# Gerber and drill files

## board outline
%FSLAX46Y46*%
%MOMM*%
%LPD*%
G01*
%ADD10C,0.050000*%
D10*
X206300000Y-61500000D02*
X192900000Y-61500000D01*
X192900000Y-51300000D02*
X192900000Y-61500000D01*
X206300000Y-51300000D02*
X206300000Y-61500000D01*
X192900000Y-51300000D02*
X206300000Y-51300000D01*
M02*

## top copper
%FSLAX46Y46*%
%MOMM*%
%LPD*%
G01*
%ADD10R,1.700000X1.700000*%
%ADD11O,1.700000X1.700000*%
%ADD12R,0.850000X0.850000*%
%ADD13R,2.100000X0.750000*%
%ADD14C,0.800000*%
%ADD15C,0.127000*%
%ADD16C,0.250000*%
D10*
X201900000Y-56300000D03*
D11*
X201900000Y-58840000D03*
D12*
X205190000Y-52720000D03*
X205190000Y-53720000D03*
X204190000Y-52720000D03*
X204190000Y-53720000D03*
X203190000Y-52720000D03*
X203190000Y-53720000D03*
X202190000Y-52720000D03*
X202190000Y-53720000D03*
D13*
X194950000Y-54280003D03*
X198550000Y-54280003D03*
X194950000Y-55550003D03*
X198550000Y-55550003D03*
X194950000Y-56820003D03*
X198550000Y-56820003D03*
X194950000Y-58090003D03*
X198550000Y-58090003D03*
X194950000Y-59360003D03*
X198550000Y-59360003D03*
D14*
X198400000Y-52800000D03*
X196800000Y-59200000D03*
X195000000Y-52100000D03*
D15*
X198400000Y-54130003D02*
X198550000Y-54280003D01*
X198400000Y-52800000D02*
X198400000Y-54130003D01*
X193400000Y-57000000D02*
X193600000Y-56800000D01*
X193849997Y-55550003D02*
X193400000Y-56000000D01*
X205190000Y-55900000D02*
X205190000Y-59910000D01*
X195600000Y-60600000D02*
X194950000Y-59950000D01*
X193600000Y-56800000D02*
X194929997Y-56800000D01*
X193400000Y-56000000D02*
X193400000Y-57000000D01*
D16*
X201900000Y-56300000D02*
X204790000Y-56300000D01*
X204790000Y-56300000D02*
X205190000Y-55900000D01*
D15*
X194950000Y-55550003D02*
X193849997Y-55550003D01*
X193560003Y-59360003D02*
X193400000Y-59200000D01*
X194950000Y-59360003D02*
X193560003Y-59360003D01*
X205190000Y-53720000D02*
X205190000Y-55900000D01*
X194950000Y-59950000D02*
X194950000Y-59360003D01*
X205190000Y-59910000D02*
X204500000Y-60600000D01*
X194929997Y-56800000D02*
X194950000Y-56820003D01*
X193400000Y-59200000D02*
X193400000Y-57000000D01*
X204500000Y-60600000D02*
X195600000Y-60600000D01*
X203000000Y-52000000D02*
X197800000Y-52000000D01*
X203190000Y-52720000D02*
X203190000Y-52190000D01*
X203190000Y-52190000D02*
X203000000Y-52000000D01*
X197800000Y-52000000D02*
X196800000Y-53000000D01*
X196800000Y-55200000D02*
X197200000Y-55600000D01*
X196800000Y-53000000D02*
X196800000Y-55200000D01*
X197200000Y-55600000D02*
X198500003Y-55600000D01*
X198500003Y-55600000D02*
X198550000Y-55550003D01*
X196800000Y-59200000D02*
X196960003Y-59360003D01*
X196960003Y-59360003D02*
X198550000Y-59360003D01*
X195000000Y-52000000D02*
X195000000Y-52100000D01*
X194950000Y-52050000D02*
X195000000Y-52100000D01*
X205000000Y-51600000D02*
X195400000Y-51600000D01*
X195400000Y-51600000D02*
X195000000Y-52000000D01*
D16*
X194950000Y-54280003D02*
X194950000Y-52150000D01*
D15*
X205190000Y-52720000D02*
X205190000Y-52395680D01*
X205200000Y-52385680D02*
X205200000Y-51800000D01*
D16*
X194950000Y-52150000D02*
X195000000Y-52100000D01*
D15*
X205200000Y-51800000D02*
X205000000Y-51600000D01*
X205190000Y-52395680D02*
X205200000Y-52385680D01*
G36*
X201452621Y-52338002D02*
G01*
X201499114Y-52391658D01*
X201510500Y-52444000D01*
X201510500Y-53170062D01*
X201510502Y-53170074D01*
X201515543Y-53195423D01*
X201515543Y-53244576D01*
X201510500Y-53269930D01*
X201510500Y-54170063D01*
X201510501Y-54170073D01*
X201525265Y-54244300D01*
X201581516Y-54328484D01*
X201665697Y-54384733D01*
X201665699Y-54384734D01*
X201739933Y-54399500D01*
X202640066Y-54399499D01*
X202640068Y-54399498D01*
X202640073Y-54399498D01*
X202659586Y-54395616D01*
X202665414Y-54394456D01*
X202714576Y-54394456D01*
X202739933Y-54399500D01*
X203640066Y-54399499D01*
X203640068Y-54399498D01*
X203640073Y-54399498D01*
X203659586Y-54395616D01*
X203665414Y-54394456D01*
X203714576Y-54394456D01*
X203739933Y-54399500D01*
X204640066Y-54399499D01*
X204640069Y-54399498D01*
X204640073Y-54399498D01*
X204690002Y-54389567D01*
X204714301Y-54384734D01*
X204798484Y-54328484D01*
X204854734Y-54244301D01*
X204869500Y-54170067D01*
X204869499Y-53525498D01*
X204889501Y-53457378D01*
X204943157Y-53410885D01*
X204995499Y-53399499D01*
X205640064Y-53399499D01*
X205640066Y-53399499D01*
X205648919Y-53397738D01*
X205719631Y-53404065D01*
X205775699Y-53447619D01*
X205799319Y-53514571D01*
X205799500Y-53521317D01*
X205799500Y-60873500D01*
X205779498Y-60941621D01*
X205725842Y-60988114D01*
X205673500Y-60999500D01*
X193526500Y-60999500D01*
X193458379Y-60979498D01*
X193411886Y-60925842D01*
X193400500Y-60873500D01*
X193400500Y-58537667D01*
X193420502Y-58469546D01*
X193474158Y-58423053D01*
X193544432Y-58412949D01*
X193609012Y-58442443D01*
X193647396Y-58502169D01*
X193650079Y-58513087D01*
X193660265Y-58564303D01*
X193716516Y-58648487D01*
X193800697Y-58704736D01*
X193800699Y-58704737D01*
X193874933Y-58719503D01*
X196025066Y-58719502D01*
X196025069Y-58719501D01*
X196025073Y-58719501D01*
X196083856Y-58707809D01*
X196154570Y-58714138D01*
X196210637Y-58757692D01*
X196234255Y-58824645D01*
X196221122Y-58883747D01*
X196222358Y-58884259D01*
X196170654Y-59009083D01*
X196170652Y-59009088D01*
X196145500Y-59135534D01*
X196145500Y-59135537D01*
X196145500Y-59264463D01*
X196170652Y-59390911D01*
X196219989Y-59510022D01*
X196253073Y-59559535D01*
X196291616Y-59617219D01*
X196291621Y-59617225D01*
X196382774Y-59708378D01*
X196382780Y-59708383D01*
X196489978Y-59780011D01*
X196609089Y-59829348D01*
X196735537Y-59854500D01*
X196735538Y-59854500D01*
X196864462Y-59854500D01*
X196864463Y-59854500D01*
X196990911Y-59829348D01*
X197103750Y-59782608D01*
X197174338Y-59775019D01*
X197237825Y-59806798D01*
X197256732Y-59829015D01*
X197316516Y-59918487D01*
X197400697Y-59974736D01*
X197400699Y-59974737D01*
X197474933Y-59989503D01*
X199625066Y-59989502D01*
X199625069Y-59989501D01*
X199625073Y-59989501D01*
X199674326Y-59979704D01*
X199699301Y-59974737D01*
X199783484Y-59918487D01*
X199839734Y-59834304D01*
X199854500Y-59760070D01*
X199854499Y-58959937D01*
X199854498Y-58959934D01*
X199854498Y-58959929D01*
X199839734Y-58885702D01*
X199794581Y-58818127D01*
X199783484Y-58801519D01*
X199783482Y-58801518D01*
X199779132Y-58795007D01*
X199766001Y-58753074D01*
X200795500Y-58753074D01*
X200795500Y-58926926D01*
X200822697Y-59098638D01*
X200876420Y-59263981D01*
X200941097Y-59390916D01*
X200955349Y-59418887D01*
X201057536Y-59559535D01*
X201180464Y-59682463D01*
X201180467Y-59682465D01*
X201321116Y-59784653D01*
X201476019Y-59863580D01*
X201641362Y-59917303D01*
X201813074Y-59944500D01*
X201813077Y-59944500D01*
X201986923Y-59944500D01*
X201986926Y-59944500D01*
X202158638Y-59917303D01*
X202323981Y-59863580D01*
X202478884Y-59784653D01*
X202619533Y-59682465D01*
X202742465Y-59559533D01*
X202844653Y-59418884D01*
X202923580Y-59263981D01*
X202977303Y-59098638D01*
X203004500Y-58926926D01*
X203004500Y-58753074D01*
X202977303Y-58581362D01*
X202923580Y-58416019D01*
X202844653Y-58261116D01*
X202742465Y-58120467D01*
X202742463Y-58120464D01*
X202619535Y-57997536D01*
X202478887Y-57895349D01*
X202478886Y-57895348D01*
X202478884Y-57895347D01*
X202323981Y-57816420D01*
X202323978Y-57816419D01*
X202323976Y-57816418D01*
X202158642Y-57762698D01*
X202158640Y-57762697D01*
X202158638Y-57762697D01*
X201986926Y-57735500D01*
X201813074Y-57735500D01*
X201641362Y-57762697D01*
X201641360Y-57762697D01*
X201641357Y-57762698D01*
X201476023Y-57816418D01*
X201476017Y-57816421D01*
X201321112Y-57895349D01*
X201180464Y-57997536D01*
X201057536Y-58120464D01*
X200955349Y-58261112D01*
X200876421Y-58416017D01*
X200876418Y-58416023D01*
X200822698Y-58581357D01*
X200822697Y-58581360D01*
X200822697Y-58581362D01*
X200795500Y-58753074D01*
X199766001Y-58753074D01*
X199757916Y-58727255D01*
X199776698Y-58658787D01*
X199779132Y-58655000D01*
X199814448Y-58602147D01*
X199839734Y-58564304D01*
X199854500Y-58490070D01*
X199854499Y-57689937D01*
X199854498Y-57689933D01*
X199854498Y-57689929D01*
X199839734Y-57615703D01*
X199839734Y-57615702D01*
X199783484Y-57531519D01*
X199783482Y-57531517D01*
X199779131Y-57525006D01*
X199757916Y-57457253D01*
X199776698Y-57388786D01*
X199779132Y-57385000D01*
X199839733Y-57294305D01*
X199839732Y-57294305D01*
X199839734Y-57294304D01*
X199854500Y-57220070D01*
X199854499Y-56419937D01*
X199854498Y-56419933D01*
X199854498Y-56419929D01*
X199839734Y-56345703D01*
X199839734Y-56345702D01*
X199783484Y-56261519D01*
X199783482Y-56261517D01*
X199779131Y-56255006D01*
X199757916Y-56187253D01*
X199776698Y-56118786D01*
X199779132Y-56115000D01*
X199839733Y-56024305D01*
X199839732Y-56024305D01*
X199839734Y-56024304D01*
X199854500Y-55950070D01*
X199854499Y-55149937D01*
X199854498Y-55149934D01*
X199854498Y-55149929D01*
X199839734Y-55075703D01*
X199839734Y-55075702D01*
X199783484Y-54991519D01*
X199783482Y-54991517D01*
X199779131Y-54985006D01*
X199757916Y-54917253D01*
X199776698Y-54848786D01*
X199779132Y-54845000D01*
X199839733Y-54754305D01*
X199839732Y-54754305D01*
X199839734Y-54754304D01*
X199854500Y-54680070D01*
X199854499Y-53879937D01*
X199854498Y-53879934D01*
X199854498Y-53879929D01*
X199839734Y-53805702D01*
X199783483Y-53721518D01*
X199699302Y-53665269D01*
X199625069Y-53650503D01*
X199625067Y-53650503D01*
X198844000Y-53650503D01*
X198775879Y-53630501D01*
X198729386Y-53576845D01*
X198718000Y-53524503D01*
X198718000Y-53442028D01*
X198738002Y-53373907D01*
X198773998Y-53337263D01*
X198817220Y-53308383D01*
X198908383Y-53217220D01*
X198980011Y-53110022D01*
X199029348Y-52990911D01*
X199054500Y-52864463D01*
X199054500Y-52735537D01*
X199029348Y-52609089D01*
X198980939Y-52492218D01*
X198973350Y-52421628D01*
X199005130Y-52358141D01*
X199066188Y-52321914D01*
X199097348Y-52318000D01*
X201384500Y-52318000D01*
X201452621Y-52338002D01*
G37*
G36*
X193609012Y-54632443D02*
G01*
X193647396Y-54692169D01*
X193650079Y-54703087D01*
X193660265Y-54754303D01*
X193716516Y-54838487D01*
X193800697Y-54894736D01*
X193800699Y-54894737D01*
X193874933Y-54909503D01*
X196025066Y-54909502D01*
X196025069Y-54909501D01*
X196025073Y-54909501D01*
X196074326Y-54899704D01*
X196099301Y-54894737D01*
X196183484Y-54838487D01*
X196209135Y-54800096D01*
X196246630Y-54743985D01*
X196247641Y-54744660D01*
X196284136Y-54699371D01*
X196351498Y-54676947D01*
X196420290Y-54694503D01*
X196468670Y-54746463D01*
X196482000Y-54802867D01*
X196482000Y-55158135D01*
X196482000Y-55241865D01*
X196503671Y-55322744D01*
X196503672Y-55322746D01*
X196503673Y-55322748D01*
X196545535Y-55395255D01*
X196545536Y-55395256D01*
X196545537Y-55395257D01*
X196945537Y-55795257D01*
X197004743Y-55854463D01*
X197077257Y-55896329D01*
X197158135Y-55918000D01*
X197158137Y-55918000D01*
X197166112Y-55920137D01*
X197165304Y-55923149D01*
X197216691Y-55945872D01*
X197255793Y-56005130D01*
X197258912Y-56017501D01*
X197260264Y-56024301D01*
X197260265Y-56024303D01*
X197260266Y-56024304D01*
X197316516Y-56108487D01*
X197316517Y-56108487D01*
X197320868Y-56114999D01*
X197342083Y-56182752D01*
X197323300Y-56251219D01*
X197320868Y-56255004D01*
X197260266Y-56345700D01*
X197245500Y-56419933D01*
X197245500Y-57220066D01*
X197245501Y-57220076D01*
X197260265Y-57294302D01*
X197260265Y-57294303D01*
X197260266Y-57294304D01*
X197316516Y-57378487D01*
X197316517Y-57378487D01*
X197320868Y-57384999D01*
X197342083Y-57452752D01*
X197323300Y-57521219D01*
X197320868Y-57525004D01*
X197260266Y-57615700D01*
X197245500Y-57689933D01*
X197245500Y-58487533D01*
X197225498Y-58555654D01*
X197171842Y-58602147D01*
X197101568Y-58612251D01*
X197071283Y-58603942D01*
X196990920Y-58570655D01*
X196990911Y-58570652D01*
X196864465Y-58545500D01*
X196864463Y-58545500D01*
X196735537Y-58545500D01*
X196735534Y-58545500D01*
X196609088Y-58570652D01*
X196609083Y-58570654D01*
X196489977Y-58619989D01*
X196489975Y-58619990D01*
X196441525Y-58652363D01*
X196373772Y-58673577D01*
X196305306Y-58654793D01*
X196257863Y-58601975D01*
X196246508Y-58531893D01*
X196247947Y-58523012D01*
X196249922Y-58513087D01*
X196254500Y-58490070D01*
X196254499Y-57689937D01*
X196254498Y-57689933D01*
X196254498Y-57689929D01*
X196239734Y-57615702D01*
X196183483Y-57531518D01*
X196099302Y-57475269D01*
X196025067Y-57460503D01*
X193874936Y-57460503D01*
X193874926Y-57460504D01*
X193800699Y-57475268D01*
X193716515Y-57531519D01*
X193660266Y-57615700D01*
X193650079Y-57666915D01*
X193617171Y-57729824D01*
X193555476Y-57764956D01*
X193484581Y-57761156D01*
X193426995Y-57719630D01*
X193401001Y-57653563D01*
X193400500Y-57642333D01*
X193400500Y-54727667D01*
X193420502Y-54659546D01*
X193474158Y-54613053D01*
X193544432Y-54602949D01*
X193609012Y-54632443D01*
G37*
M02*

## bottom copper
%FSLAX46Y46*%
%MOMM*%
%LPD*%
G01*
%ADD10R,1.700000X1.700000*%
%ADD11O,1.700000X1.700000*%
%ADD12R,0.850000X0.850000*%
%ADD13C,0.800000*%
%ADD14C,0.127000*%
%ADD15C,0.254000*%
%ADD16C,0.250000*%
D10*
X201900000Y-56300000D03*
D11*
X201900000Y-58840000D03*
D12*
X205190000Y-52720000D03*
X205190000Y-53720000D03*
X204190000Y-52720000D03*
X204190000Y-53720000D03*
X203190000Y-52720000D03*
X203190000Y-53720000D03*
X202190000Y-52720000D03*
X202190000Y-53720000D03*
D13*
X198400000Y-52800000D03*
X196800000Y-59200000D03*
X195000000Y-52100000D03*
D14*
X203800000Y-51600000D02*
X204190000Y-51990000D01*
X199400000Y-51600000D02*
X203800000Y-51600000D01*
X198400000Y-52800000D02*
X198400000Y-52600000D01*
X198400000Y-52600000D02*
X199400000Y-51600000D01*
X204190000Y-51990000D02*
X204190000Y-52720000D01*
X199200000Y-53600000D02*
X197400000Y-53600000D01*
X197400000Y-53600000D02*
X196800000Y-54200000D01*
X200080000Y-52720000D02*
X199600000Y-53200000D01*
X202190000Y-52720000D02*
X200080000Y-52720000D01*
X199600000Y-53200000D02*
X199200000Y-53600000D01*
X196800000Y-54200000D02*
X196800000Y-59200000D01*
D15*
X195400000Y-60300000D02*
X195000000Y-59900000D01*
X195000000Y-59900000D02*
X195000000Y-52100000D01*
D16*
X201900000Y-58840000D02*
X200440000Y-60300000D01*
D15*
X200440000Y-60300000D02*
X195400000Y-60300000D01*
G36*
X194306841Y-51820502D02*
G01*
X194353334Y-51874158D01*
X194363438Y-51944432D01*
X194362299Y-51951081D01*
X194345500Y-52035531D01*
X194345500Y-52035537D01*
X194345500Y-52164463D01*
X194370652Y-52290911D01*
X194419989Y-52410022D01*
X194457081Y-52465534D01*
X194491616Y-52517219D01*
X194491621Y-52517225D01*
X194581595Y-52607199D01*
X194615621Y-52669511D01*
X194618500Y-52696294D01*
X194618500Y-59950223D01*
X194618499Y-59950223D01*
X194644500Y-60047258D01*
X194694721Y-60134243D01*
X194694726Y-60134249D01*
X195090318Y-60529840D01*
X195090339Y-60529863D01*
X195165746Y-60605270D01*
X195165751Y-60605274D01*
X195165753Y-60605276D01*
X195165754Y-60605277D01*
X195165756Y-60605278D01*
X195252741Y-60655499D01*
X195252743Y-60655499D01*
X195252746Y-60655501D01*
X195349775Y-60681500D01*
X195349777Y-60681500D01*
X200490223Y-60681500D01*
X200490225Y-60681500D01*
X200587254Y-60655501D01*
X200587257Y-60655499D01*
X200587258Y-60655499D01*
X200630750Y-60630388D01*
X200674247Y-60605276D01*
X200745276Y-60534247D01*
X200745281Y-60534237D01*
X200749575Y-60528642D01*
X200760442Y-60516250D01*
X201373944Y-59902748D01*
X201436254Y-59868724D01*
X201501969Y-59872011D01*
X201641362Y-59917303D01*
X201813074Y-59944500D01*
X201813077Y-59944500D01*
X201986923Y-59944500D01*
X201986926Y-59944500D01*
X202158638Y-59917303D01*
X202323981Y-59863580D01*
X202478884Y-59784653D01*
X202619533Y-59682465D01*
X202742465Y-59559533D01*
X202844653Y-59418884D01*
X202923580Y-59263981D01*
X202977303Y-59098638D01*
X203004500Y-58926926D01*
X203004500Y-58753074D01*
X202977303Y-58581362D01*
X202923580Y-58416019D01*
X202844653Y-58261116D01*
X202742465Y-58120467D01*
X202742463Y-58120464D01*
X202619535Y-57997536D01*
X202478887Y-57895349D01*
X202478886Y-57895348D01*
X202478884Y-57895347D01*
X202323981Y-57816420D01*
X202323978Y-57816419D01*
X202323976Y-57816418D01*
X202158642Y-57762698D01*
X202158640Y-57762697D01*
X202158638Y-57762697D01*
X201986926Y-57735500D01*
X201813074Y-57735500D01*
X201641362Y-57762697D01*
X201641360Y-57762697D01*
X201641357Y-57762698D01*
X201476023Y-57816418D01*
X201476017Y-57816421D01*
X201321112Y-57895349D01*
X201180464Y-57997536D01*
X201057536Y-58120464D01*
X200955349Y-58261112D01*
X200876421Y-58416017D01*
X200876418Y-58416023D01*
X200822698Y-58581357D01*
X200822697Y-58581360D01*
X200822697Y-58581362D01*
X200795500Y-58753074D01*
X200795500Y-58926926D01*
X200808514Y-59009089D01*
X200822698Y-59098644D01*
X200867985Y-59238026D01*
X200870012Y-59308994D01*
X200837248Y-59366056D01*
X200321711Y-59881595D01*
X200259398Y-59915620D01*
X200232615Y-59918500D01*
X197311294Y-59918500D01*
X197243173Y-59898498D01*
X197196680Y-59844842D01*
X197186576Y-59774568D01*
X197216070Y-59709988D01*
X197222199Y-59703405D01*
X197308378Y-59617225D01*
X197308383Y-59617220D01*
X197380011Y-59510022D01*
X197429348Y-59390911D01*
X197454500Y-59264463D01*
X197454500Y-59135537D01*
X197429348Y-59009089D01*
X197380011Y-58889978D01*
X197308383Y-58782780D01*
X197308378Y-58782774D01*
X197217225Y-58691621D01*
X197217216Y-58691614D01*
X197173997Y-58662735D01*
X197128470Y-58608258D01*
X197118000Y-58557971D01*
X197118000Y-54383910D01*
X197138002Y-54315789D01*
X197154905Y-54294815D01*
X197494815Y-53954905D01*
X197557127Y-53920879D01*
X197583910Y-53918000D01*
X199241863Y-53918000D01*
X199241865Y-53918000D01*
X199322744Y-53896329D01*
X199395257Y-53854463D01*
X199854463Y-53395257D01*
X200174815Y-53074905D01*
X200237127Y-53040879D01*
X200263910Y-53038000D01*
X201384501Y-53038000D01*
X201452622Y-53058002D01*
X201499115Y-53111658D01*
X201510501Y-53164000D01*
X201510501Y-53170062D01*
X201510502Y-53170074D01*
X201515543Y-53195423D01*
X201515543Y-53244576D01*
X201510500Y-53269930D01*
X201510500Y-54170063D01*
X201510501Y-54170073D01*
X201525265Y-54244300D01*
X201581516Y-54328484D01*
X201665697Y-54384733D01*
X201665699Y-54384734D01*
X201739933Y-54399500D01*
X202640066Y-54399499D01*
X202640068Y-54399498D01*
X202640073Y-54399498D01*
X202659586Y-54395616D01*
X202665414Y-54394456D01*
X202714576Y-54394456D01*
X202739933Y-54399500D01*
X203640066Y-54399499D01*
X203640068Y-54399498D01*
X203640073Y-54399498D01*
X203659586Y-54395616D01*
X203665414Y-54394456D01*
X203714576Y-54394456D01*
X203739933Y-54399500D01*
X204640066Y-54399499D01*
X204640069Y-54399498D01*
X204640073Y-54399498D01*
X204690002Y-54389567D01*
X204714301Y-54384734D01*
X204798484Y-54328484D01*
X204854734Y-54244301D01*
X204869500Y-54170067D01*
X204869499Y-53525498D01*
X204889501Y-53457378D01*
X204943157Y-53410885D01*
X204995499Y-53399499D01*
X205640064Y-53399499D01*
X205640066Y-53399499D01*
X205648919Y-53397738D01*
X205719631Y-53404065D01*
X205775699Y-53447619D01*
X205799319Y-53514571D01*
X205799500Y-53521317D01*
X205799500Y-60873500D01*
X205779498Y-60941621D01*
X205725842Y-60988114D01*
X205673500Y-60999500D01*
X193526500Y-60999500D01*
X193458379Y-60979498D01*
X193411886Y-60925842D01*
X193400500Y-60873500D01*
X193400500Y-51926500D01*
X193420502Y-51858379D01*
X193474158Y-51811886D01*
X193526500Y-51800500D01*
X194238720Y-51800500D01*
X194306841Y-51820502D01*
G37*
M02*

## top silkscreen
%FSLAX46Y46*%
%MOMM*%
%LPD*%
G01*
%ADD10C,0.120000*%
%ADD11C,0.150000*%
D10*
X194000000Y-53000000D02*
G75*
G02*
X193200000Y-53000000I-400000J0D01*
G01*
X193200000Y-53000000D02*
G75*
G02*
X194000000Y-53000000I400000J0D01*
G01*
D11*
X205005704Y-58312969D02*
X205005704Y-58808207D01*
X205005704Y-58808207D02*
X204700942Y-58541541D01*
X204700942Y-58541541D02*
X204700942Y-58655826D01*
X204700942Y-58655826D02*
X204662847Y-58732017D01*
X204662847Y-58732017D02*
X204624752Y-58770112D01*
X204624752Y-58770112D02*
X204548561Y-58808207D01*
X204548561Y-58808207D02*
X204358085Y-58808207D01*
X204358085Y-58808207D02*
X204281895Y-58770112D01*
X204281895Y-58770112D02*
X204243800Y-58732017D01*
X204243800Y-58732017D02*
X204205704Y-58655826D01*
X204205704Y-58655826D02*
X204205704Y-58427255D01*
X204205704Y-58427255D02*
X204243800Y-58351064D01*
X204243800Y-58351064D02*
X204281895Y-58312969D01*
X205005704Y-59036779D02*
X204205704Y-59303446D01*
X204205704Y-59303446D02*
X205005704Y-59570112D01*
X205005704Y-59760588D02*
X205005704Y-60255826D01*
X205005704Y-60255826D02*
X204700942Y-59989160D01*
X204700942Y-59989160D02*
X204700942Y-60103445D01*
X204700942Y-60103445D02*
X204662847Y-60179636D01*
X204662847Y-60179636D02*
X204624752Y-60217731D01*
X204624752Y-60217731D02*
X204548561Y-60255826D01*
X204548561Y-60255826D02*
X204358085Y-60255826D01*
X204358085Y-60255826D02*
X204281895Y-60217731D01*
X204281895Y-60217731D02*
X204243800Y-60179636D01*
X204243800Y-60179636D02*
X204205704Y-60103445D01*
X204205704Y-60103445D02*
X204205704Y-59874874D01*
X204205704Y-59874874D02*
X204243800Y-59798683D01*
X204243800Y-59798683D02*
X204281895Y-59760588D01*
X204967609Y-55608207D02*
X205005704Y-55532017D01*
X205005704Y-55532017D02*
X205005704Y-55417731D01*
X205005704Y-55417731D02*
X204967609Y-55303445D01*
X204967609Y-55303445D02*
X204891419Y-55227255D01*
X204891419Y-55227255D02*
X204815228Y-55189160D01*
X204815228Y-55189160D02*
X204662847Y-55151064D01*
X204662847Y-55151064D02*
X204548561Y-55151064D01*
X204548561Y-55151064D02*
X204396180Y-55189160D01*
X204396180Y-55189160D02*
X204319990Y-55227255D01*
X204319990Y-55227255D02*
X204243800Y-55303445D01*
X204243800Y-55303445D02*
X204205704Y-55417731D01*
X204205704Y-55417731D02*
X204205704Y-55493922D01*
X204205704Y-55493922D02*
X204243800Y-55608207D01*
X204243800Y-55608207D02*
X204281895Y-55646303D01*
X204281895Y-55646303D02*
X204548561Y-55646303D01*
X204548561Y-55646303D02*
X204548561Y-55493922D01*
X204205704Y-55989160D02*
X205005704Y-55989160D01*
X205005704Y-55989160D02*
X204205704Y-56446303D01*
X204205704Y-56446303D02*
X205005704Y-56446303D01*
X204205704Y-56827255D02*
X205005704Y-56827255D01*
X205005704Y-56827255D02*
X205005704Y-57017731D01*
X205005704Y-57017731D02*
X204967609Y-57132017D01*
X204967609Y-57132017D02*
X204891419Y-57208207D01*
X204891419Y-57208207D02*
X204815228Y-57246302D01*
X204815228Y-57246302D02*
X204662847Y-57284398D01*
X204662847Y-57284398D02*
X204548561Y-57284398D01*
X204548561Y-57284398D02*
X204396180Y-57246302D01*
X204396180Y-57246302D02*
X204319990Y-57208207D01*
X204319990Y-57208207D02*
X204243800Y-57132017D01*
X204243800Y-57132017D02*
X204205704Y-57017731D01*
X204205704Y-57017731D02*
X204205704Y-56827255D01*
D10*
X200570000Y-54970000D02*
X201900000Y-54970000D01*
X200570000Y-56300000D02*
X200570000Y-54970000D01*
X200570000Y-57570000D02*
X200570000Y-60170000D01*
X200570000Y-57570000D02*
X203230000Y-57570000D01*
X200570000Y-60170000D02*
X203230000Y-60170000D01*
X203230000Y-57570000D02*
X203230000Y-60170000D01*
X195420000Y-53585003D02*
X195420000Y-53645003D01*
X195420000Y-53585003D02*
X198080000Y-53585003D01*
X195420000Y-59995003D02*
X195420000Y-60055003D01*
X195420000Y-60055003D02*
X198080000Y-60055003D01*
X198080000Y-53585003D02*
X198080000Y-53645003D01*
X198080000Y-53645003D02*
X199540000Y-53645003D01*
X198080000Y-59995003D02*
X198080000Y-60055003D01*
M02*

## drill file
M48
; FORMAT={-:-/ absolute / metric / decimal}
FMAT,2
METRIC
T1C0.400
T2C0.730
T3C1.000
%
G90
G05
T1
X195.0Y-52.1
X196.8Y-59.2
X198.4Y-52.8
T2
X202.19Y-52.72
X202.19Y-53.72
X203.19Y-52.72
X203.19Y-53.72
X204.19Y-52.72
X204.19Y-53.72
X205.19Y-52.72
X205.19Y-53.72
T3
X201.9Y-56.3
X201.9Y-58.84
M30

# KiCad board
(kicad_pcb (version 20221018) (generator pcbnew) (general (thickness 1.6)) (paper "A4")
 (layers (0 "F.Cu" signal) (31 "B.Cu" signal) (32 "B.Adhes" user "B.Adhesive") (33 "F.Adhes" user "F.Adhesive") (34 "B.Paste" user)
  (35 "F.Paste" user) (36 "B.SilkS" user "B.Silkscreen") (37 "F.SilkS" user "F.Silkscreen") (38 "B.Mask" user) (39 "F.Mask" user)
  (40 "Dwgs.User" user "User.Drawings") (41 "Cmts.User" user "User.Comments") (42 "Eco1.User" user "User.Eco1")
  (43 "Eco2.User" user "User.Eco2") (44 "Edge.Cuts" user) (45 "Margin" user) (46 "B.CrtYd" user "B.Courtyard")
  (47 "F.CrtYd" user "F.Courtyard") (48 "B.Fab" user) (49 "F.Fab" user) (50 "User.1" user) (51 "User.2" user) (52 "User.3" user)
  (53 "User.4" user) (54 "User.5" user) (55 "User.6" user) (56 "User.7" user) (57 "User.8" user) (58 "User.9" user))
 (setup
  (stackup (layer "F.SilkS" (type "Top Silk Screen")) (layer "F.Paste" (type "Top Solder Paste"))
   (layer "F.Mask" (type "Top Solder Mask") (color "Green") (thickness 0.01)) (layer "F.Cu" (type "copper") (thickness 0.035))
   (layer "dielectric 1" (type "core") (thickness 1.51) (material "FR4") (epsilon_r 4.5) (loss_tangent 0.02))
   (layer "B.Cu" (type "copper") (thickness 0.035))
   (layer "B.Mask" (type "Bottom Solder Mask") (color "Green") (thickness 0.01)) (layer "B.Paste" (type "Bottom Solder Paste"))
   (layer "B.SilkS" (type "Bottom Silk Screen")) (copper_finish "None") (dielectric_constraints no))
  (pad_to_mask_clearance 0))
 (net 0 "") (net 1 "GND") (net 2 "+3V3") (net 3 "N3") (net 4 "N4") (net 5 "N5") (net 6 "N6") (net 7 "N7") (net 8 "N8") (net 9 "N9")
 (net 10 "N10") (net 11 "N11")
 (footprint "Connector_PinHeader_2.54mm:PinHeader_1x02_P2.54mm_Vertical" (layer "F.Cu") (at 201.9 56.3)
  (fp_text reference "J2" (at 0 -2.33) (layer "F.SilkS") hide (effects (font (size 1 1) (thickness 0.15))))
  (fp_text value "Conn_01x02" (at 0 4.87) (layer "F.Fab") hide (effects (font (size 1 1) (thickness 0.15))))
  (fp_line (start -1.33 -1.33) (end 0 -1.33) (stroke (width 0.12) (type solid)) (layer "F.SilkS"))
  (fp_line (start -1.33 0) (end -1.33 -1.33) (stroke (width 0.12) (type solid)) (layer "F.SilkS"))
  (fp_line (start -1.33 1.27) (end -1.33 3.87) (stroke (width 0.12) (type solid)) (layer "F.SilkS"))
  (fp_line (start -1.33 1.27) (end 1.33 1.27) (stroke (width 0.12) (type solid)) (layer "F.SilkS"))
  (fp_line (start -1.33 3.87) (end 1.33 3.87) (stroke (width 0.12) (type solid)) (layer "F.SilkS"))
  (fp_line (start 1.33 1.27) (end 1.33 3.87) (stroke (width 0.12) (type solid)) (layer "F.SilkS"))
  (pad "1" thru_hole rect (at 0 0) (size 1.7 1.7) (drill 1) (layers "*.Cu" "*.Mask") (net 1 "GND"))
  (pad "2" thru_hole oval (at 0 2.54) (size 1.7 1.7) (drill 1) (layers "*.Cu" "*.Mask") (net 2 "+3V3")))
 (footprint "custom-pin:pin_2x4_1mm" (layer "F.Cu") (at 203.69 53.22)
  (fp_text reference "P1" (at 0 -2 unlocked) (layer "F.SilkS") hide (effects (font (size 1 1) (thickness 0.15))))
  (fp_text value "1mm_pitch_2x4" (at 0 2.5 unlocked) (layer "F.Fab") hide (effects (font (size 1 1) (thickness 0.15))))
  (pad "1" thru_hole rect (at 1.5 -0.5) (size 0.85 0.85) (drill 0.73) (layers "*.Cu" "*.Mask") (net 2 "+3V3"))
  (pad "2" thru_hole rect (at 1.5 0.5) (size 0.85 0.85) (drill 0.73) (layers "*.Cu" "*.Mask") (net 1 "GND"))
  (pad "3" thru_hole rect (at 0.5 -0.5) (size 0.85 0.85) (drill 0.73) (layers "*.Cu" "*.Mask") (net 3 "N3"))
  (pad "4" thru_hole rect (at 0.5 0.5) (size 0.85 0.85) (drill 0.73) (layers "*.Cu" "*.Mask") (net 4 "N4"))
  (pad "5" thru_hole rect (at -0.5 -0.5) (size 0.85 0.85) (drill 0.73) (layers "*.Cu" "*.Mask") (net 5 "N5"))
  (pad "6" thru_hole rect (at -0.5 0.5) (size 0.85 0.85) (drill 0.73) (layers "*.Cu" "*.Mask") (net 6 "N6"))
  (pad "7" thru_hole rect (at -1.5 -0.5) (size 0.85 0.85) (drill 0.73) (layers "*.Cu" "*.Mask") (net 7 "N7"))
  (pad "8" thru_hole rect (at -1.5 0.5) (size 0.85 0.85) (drill 0.73) (layers "*.Cu" "*.Mask") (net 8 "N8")))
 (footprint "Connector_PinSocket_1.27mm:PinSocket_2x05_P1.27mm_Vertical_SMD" (layer "F.Cu") (at 196.75 56.820003)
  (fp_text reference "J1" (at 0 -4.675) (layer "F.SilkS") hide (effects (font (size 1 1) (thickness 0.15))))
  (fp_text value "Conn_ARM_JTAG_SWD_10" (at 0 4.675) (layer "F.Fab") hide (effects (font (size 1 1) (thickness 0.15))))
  (fp_line (start -1.33 -3.235) (end -1.33 -3.175) (stroke (width 0.12) (type solid)) (layer "F.SilkS"))
  (fp_line (start -1.33 -3.235) (end 1.33 -3.235) (stroke (width 0.12) (type solid)) (layer "F.SilkS"))
  (fp_line (start -1.33 3.175) (end -1.33 3.235) (stroke (width 0.12) (type solid)) (layer "F.SilkS"))
  (fp_line (start -1.33 3.235) (end 1.33 3.235) (stroke (width 0.12) (type solid)) (layer "F.SilkS"))
  (fp_line (start 1.33 -3.235) (end 1.33 -3.175) (stroke (width 0.12) (type solid)) (layer "F.SilkS"))
  (fp_line (start 1.33 -3.175) (end 2.79 -3.175) (stroke (width 0.12) (type solid)) (layer "F.SilkS"))
  (fp_line (start 1.33 3.175) (end 1.33 3.235) (stroke (width 0.12) (type solid)) (layer "F.SilkS"))
  (pad "1" smd rect (at -1.8 -2.54) (size 2.1 0.75) (layers "F.Cu" "F.Paste" "F.Mask") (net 2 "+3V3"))
  (pad "2" smd rect (at 1.8 -2.54) (size 2.1 0.75) (layers "F.Cu" "F.Paste" "F.Mask") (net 3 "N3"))
  (pad "3" smd rect (at -1.8 -1.27) (size 2.1 0.75) (layers "F.Cu" "F.Paste" "F.Mask") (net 1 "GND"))
  (pad "4" smd rect (at 1.8 -1.27) (size 2.1 0.75) (layers "F.Cu" "F.Paste" "F.Mask") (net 5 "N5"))
  (pad "5" smd rect (at -1.8 0) (size 2.1 0.75) (layers "F.Cu" "F.Paste" "F.Mask") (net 1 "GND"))
  (pad "6" smd rect (at 1.8 0) (size 2.1 0.75) (layers "F.Cu" "F.Paste" "F.Mask") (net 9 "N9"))
  (pad "7" smd rect (at -1.8 1.27) (size 2.1 0.75) (layers "F.Cu" "F.Paste" "F.Mask") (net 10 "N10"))
  (pad "8" smd rect (at 1.8 1.27) (size 2.1 0.75) (layers "F.Cu" "F.Paste" "F.Mask") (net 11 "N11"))
  (pad "9" smd rect (at -1.8 2.54) (size 2.1 0.75) (layers "F.Cu" "F.Paste" "F.Mask") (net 1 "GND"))
  (pad "10" smd rect (at 1.8 2.54) (size 2.1 0.75) (layers "F.Cu" "F.Paste" "F.Mask") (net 7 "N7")))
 (gr_circle (center 193.6 53) (end 194 53) (stroke (width 0.12) (type solid)) (fill none) (layer "F.SilkS"))
 (gr_line (start 206.3 61.5) (end 192.9 61.5) (stroke (width 0.05) (type solid)) (layer "Edge.Cuts"))
 (gr_line (start 192.9 51.3) (end 192.9 61.5) (stroke (width 0.05) (type solid)) (layer "Edge.Cuts"))
 (gr_line (start 206.3 51.3) (end 206.3 61.5) (stroke (width 0.05) (type solid)) (layer "Edge.Cuts"))
 (gr_line (start 192.9 51.3) (end 206.3 51.3) (stroke (width 0.05) (type solid)) (layer "Edge.Cuts"))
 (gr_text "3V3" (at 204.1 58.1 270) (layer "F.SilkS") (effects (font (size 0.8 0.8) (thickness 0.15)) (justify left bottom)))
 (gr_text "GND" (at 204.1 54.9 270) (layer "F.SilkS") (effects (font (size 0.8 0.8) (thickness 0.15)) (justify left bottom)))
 (segment (start 198.4 54.130003) (end 198.55 54.280003) (width 0.127) (layer "F.Cu") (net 3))
 (segment (start 198.4 52.8) (end 198.4 54.130003) (width 0.127) (layer "F.Cu") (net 3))
 (via (at 198.4 52.8) (size 0.8) (drill 0.4) (layers "F.Cu" "B.Cu") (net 3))
 (segment (start 203.8 51.6) (end 204.19 51.99) (width 0.127) (layer "B.Cu") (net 3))
 (segment (start 199.4 51.6) (end 203.8 51.6) (width 0.127) (layer "B.Cu") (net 3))
 (segment (start 198.4 52.8) (end 198.4 52.6) (width 0.127) (layer "B.Cu") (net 3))
 (segment (start 198.4 52.6) (end 199.4 51.6) (width 0.127) (layer "B.Cu") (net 3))
 (segment (start 204.19 51.99) (end 204.19 52.72) (width 0.127) (layer "B.Cu") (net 3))
 (segment (start 193.4 57) (end 193.6 56.8) (width 0.127) (layer "F.Cu") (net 1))
 (segment (start 193.849997 55.550003) (end 193.4 56) (width 0.127) (layer "F.Cu") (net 1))
 (segment (start 205.19 55.9) (end 205.19 59.91) (width 0.127) (layer "F.Cu") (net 1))
 (segment (start 195.6 60.6) (end 194.95 59.95) (width 0.127) (layer "F.Cu") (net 1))
 (segment (start 193.6 56.8) (end 194.929997 56.8) (width 0.127) (layer "F.Cu") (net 1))
 (segment (start 193.4 56) (end 193.4 57) (width 0.127) (layer "F.Cu") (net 1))
 (segment (start 201.9 56.3) (end 204.79 56.3) (width 0.25) (layer "F.Cu") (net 1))
 (segment (start 204.79 56.3) (end 205.19 55.9) (width 0.25) (layer "F.Cu") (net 1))
 (segment (start 194.95 55.550003) (end 193.849997 55.550003) (width 0.127) (layer "F.Cu") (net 1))
 (segment (start 193.560003 59.360003) (end 193.4 59.2) (width 0.127) (layer "F.Cu") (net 1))
 (segment (start 194.95 59.360003) (end 193.560003 59.360003) (width 0.127) (layer "F.Cu") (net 1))
 (segment (start 205.19 53.72) (end 205.19 55.9) (width 0.127) (layer "F.Cu") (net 1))
 (segment (start 194.95 59.95) (end 194.95 59.360003) (width 0.127) (layer "F.Cu") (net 1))
 (segment (start 205.19 59.91) (end 204.5 60.6) (width 0.127) (layer "F.Cu") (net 1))
 (segment (start 194.929997 56.8) (end 194.95 56.820003) (width 0.127) (layer "F.Cu") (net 1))
 (segment (start 193.4 59.2) (end 193.4 57) (width 0.127) (layer "F.Cu") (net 1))
 (segment (start 204.5 60.6) (end 195.6 60.6) (width 0.127) (layer "F.Cu") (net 1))
 (segment (start 203 52) (end 197.8 52) (width 0.127) (layer "F.Cu") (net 5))
 (segment (start 203.19 52.72) (end 203.19 52.19) (width 0.127) (layer "F.Cu") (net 5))
 (segment (start 203.19 52.19) (end 203 52) (width 0.127) (layer "F.Cu") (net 5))
 (segment (start 197.8 52) (end 196.8 53) (width 0.127) (layer "F.Cu") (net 5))
 (segment (start 196.8 55.2) (end 197.2 55.6) (width 0.127) (layer "F.Cu") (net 5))
 (segment (start 196.8 53) (end 196.8 55.2) (width 0.127) (layer "F.Cu") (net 5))
 (segment (start 197.2 55.6) (end 198.500003 55.6) (width 0.127) (layer "F.Cu") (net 5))
 (segment (start 198.500003 55.6) (end 198.55 55.550003) (width 0.127) (layer "F.Cu") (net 5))
 (segment (start 196.8 59.2) (end 196.960003 59.360003) (width 0.127) (layer "F.Cu") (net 7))
 (segment (start 196.960003 59.360003) (end 198.55 59.360003) (width 0.127) (layer "F.Cu") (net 7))
 (via (at 196.8 59.2) (size 0.8) (drill 0.4) (layers "F.Cu" "B.Cu") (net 7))
 (segment (start 199.2 53.6) (end 197.4 53.6) (width 0.127) (layer "B.Cu") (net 7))
 (segment (start 197.4 53.6) (end 196.8 54.2) (width 0.127) (layer "B.Cu") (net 7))
 (segment (start 200.08 52.72) (end 199.6 53.2) (width 0.127) (layer "B.Cu") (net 7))
 (segment (start 202.19 52.72) (end 200.08 52.72) (width 0.127) (layer "B.Cu") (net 7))
 (segment (start 199.6 53.2) (end 199.2 53.6) (width 0.127) (layer "B.Cu") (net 7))
 (segment (start 196.8 54.2) (end 196.8 59.2) (width 0.127) (layer "B.Cu") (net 7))
 (segment (start 195 52) (end 195 52.1) (width 0.127) (layer "F.Cu") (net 2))
 (segment (start 194.95 52.05) (end 195 52.1) (width 0.127) (layer "F.Cu") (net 2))
 (segment (start 205 51.6) (end 195.4 51.6) (width 0.127) (layer "F.Cu") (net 2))
 (segment (start 195.4 51.6) (end 195 52) (width 0.127) (layer "F.Cu") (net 2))
 (segment (start 194.95 54.280003) (end 194.95 52.15) (width 0.25) (layer "F.Cu") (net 2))
 (segment (start 205.19 52.72) (end 205.19 52.39568) (width 0.127) (layer "F.Cu") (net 2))
 (segment (start 205.2 52.38568) (end 205.2 51.8) (width 0.127) (layer "F.Cu") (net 2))
 (segment (start 194.95 52.15) (end 195 52.1) (width 0.25) (layer "F.Cu") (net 2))
 (segment (start 205.2 51.8) (end 205 51.6) (width 0.127) (layer "F.Cu") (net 2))
 (segment (start 205.19 52.39568) (end 205.2 52.38568) (width 0.127) (layer "F.Cu") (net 2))
 (via (at 195 52.1) (size 0.8) (drill 0.4) (layers "F.Cu" "B.Cu") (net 2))
 (segment (start 195.4 60.3) (end 195 59.9) (width 0.254) (layer "B.Cu") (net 2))
 (segment (start 195 59.9) (end 195 52.1) (width 0.254) (layer "B.Cu") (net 2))
 (segment (start 201.9 58.84) (end 200.44 60.3) (width 0.25) (layer "B.Cu") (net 2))
 (segment (start 200.44 60.3) (end 195.4 60.3) (width 0.254) (layer "B.Cu") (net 2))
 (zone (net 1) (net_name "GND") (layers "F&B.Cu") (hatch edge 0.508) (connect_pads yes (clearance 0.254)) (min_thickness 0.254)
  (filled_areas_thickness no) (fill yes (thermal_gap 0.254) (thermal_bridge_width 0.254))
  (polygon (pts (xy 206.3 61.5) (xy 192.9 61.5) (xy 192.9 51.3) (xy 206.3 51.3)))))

